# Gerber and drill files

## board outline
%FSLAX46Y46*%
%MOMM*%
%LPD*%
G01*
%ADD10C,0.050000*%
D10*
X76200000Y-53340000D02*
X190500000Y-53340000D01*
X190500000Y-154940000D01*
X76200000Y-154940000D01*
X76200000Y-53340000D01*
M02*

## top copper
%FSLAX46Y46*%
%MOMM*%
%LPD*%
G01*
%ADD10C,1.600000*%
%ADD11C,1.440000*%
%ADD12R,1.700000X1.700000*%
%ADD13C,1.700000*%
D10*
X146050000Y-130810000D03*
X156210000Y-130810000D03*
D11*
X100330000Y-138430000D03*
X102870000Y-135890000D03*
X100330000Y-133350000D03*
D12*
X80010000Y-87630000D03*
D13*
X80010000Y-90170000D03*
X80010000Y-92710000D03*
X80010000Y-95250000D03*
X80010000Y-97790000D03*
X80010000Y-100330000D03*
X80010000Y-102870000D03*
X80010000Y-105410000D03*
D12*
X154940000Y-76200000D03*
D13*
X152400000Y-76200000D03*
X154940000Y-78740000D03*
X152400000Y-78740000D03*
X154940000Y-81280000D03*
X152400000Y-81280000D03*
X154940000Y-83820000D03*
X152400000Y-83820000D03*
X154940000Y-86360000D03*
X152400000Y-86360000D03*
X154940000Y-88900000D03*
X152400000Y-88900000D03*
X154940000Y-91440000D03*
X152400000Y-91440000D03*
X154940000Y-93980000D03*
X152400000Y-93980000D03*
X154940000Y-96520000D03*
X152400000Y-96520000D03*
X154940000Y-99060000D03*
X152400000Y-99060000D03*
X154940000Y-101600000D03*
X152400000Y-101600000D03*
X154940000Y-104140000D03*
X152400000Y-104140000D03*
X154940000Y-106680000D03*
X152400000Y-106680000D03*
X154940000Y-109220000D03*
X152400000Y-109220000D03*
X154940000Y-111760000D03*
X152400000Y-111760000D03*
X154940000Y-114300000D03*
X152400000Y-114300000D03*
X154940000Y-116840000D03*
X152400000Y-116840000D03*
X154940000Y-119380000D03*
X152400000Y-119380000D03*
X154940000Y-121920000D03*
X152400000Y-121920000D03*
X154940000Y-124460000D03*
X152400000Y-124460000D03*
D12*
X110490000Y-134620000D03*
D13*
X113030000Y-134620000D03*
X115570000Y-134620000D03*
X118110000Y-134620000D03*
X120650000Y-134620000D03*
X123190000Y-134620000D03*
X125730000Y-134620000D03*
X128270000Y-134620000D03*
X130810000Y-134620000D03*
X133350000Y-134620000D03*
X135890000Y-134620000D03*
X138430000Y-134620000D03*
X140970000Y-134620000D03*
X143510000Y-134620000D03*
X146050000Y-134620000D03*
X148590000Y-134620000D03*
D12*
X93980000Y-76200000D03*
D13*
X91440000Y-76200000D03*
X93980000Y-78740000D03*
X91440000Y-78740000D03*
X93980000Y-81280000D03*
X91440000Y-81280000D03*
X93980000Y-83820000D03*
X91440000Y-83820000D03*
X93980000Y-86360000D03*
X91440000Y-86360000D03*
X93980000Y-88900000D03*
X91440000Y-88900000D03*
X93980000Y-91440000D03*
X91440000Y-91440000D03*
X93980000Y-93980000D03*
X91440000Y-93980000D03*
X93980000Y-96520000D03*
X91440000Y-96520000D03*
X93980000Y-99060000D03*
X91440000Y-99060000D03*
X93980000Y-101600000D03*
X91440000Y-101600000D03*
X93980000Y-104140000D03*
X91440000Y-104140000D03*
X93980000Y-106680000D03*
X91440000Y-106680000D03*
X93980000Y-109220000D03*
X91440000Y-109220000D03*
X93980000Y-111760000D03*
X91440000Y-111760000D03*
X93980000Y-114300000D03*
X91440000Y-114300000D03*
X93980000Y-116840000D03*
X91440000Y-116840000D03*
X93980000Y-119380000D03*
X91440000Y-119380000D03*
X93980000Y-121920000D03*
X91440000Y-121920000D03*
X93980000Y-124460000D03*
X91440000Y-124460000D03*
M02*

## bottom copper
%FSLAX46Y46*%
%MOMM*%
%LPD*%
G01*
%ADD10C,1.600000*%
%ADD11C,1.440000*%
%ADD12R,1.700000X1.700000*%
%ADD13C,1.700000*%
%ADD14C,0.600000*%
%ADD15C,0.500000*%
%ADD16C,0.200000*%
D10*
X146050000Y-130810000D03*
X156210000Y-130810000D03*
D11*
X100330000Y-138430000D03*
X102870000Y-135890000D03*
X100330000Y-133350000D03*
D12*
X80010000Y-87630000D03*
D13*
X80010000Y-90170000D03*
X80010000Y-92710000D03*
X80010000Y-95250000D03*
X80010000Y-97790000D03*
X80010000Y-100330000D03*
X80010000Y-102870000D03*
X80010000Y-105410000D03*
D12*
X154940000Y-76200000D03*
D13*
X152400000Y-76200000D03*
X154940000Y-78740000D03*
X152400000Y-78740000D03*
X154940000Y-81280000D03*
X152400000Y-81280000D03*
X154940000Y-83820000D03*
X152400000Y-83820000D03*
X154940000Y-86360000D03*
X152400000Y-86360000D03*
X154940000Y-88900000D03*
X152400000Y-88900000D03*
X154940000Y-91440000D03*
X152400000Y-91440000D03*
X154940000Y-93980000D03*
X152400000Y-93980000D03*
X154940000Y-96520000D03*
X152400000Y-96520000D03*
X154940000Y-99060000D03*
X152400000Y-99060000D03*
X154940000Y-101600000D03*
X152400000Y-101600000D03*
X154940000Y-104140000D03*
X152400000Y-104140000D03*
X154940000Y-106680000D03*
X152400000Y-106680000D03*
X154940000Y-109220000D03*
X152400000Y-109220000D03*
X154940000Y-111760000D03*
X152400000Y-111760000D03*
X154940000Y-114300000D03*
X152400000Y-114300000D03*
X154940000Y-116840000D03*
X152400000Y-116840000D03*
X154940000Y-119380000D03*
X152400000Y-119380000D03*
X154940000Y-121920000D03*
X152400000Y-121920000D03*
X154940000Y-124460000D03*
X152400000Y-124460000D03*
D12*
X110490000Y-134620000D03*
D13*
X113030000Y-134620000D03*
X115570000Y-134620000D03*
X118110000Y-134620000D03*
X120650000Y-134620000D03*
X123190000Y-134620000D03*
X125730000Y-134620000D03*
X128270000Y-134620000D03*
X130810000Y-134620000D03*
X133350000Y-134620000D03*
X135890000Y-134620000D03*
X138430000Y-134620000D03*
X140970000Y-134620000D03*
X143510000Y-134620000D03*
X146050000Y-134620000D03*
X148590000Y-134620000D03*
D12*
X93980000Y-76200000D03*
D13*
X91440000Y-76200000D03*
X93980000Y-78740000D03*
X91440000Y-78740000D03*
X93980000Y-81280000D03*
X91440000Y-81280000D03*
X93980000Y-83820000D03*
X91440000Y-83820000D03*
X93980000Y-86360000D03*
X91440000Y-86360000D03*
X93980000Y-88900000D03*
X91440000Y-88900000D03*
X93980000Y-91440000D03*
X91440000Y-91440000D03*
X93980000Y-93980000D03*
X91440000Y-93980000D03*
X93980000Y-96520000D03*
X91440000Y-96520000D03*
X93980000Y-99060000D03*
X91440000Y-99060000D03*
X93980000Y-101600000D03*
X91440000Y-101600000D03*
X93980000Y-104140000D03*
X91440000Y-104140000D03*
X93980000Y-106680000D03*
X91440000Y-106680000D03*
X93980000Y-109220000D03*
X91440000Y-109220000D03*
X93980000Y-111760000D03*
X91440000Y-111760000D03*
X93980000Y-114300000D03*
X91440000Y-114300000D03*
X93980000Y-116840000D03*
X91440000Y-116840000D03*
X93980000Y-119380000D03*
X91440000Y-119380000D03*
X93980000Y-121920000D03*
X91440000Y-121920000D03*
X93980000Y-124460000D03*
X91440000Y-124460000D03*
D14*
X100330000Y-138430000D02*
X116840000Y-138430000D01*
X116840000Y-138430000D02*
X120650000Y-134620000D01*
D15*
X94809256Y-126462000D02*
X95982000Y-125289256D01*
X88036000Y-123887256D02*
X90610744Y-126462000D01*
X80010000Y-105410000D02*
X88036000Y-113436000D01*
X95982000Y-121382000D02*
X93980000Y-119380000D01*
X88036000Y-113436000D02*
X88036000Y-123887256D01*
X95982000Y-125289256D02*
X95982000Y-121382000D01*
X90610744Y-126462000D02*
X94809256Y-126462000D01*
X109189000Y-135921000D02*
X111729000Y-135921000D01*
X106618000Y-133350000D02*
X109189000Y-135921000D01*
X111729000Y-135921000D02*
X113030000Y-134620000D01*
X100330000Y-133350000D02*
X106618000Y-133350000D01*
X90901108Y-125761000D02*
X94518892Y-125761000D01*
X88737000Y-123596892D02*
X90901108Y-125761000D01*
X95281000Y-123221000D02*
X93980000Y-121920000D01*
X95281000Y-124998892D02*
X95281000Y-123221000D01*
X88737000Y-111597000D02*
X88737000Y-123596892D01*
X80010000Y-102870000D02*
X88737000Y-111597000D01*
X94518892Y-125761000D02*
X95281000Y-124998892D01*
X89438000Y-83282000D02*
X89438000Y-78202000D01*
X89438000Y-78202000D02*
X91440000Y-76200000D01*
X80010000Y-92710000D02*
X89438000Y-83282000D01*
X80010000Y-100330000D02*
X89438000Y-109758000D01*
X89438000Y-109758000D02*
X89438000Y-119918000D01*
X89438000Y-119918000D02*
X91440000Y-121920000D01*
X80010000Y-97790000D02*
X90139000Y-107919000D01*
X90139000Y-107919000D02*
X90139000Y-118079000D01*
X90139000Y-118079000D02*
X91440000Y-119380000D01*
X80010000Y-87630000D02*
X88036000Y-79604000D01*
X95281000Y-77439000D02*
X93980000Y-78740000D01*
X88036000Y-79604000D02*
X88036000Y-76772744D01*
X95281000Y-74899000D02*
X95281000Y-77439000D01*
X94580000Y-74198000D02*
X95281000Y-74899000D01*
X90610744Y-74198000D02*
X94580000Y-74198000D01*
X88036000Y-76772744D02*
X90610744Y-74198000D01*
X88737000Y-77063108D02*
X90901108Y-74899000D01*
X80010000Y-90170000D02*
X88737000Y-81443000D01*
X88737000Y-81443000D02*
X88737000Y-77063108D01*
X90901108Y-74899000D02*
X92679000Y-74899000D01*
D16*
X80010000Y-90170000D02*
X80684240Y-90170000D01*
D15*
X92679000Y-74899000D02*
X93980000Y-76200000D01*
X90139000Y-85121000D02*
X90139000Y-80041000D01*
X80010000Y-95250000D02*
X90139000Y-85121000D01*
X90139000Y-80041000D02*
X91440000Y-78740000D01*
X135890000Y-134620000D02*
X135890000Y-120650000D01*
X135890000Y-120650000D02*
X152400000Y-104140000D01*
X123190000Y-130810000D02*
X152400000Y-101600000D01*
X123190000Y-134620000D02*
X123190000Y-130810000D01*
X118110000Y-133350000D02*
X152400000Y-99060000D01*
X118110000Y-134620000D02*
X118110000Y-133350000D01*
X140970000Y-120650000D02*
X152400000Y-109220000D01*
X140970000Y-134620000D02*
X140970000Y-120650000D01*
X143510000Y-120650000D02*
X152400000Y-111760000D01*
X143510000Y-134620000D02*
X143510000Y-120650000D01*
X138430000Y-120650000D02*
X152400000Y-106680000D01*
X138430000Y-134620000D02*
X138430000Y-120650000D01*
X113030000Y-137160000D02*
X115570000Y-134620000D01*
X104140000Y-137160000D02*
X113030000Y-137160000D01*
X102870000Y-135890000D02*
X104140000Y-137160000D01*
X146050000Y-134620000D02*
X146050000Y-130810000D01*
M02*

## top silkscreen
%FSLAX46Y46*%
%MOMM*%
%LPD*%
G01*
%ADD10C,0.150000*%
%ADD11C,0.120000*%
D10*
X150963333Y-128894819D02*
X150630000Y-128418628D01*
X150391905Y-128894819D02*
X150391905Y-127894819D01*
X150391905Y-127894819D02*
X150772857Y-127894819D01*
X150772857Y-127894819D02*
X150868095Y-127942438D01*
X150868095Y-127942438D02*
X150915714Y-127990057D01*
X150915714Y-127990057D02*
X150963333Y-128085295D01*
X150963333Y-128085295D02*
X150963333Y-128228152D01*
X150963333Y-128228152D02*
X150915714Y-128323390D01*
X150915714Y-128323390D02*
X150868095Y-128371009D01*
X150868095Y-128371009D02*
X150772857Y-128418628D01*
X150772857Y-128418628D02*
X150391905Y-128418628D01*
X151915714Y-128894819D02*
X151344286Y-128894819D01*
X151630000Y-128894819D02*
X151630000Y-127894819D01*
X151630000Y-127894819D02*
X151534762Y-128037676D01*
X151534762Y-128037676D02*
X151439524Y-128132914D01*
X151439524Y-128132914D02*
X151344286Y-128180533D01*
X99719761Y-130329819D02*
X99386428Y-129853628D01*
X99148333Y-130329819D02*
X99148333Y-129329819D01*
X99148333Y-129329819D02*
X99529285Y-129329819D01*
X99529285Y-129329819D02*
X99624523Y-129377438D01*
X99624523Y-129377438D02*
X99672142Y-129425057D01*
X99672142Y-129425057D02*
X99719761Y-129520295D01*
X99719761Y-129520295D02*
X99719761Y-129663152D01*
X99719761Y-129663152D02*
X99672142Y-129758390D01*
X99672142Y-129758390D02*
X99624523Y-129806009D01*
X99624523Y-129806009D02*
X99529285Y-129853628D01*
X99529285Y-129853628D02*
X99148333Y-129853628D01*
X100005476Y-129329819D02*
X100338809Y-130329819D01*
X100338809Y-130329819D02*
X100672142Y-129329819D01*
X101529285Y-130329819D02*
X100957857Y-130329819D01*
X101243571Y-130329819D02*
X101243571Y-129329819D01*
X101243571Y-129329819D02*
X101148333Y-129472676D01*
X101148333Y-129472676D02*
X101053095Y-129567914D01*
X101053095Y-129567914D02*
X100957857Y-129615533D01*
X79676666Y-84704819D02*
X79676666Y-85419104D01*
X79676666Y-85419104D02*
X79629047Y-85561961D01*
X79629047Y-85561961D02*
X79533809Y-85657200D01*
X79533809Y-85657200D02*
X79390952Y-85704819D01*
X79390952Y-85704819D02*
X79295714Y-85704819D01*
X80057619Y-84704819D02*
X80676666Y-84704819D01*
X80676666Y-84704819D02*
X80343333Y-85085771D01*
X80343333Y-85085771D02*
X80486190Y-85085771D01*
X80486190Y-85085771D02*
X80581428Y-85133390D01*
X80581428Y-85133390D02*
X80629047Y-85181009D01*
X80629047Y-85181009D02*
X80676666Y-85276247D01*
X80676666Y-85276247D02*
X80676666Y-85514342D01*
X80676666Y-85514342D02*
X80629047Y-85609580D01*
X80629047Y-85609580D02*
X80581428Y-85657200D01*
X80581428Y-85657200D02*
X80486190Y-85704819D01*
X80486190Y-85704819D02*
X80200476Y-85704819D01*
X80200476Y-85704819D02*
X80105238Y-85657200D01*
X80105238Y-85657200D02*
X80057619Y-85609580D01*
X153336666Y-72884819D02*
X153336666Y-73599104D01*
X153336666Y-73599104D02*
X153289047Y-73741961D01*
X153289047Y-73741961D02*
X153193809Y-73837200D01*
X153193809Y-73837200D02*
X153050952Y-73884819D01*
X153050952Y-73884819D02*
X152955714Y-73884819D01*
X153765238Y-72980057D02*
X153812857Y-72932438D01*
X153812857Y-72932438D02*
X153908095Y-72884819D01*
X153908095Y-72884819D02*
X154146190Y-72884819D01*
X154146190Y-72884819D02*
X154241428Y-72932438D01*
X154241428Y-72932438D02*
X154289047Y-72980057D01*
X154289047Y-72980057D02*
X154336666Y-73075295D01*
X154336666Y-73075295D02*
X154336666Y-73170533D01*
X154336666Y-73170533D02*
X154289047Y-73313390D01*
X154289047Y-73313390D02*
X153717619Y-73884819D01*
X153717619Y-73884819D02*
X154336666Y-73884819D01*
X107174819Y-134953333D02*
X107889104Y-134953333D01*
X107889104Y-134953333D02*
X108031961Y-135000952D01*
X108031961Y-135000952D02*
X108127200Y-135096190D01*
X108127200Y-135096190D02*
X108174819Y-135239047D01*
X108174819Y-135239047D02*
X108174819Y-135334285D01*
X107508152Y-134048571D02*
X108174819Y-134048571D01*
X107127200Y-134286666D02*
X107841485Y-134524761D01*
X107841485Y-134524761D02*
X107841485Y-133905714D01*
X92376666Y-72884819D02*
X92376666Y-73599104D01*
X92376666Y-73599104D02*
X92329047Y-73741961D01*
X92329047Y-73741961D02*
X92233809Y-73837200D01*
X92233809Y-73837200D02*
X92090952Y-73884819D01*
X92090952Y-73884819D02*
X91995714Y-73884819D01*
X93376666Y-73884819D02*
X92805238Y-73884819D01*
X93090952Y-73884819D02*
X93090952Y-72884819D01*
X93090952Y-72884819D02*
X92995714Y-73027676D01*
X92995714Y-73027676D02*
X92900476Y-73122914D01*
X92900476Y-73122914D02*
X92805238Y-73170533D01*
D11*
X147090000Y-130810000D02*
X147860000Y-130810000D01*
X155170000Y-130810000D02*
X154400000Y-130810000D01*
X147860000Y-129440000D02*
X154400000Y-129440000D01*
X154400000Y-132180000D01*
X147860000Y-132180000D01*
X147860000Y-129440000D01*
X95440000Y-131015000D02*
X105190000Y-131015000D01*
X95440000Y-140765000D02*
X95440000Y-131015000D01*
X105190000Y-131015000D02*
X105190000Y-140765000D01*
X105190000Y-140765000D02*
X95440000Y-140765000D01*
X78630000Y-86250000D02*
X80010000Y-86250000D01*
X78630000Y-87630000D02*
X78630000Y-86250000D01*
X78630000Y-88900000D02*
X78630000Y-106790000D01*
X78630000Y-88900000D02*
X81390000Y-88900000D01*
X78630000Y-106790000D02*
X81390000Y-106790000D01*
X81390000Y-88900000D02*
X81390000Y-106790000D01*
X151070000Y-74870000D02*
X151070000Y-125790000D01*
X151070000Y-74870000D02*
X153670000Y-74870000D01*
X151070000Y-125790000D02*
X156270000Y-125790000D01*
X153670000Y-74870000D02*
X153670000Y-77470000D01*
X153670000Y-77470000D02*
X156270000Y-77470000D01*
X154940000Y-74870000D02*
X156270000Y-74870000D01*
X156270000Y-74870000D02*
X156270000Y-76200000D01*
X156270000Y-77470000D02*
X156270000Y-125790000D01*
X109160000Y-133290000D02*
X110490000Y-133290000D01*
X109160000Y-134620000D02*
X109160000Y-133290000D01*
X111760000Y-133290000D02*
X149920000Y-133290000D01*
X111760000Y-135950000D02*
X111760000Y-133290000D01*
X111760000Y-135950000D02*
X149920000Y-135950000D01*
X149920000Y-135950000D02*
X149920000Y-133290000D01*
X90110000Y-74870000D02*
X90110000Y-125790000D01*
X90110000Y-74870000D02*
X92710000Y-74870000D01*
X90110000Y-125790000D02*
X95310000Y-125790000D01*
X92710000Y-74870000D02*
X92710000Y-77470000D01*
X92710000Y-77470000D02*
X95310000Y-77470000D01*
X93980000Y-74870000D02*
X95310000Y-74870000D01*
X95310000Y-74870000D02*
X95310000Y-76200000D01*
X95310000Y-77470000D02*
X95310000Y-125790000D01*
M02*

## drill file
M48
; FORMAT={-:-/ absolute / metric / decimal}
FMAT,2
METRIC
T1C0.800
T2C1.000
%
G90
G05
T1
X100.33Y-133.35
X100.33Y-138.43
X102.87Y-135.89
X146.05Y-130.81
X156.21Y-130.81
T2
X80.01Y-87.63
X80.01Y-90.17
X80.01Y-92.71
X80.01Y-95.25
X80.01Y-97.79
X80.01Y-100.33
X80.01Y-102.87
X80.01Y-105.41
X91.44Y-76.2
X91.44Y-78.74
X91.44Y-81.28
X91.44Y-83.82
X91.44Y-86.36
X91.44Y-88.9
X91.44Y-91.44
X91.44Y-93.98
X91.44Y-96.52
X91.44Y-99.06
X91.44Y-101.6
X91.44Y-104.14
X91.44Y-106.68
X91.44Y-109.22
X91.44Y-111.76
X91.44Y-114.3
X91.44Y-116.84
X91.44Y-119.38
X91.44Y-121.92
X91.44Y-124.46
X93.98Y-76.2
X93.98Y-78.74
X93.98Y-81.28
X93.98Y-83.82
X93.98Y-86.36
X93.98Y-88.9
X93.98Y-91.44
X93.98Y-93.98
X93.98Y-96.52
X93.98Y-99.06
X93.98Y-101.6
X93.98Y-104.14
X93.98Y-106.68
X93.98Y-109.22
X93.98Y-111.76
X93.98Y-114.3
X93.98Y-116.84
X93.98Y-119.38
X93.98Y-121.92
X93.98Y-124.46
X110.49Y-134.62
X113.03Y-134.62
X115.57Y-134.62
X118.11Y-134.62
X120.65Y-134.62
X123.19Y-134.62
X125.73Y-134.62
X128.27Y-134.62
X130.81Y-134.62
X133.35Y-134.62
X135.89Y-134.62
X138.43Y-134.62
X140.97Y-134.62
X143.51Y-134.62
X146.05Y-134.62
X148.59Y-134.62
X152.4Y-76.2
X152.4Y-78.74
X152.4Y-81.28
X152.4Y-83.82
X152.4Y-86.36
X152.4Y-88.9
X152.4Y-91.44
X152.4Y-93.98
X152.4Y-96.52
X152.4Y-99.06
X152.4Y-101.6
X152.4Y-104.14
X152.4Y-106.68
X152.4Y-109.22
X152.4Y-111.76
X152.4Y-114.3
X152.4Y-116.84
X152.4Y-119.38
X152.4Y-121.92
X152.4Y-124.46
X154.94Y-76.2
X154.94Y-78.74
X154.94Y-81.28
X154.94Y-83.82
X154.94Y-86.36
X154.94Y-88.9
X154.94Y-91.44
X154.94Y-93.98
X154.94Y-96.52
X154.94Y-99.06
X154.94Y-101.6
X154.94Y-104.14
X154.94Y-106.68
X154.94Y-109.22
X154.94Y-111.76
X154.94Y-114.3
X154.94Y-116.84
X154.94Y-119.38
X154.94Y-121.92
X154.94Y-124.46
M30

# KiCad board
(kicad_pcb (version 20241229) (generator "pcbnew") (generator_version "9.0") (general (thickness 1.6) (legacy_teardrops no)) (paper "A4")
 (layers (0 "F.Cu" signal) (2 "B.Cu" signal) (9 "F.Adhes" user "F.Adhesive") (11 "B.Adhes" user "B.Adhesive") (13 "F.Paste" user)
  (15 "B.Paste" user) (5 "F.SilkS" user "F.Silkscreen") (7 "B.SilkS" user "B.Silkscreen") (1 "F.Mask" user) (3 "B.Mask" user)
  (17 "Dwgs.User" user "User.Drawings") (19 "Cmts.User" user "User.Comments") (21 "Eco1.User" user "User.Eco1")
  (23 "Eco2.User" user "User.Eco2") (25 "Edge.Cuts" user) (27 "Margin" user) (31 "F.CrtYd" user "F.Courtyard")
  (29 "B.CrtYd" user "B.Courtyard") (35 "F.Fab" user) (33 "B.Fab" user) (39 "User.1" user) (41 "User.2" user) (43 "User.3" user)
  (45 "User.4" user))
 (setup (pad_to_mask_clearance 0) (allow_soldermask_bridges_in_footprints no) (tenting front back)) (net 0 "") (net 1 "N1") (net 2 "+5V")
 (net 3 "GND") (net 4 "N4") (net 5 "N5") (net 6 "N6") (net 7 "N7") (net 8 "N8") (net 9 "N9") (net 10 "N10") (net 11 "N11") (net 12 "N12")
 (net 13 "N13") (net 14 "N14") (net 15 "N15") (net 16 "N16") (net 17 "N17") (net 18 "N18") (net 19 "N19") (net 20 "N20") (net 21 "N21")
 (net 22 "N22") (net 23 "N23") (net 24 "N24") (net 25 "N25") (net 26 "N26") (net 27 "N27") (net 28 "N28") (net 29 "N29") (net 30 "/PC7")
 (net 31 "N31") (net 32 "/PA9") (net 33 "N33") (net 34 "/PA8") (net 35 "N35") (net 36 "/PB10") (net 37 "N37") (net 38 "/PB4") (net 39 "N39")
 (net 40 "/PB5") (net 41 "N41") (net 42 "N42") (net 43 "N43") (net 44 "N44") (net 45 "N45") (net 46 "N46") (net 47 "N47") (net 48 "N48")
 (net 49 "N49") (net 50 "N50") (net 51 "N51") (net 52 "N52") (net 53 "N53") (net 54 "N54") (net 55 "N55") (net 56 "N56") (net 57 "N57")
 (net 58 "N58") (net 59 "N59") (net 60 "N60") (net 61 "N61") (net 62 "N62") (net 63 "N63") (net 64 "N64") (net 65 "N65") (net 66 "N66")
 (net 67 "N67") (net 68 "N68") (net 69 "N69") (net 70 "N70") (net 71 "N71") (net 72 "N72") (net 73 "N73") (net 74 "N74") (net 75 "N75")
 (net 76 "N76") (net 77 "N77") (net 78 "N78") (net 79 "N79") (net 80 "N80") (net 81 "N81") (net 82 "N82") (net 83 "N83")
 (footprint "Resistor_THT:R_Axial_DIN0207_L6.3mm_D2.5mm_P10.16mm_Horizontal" (layer "F.Cu") (at 146.05 130.81)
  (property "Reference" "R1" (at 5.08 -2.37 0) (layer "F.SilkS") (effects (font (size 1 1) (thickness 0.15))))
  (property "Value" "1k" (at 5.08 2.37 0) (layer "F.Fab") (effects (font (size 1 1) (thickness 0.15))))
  (fp_line (start 1.04 0) (end 1.81 0) (stroke (width 0.12) (type solid)) (layer "F.SilkS"))
  (fp_line (start 9.12 0) (end 8.35 0) (stroke (width 0.12) (type solid)) (layer "F.SilkS"))
  (fp_rect (start 1.81 -1.37) (end 8.35 1.37) (stroke (width 0.12) (type solid)) (fill no) (layer "F.SilkS"))
  (pad "1" thru_hole circle (at 0 0) (size 1.6 1.6) (drill 0.8) (layers "*.Cu" "*.Mask") (remove_unused_layers no) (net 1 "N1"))
  (pad "2" thru_hole circle (at 10.16 0) (size 1.6 1.6) (drill 0.8) (layers "*.Cu" "*.Mask") (remove_unused_layers no) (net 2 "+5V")))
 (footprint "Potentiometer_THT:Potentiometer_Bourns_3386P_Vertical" (layer "F.Cu") (at 100.33 138.43)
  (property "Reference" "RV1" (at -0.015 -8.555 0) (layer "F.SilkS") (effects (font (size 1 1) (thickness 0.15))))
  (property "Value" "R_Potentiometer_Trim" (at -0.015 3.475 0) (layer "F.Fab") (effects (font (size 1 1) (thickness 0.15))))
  (fp_line (start -4.89 -7.415) (end 4.86 -7.415) (stroke (width 0.12) (type solid)) (layer "F.SilkS"))
  (fp_line (start -4.89 2.335) (end -4.89 -7.415) (stroke (width 0.12) (type solid)) (layer "F.SilkS"))
  (fp_line (start 4.86 -7.415) (end 4.86 2.335) (stroke (width 0.12) (type solid)) (layer "F.SilkS"))
  (fp_line (start 4.86 2.335) (end -4.89 2.335) (stroke (width 0.12) (type solid)) (layer "F.SilkS"))
  (pad "1" thru_hole circle (at 0 0) (size 1.44 1.44) (drill 0.8) (layers "*.Cu" "*.Mask") (remove_unused_layers no) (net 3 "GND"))
  (pad "2" thru_hole circle (at 2.54 -2.54) (size 1.44 1.44) (drill 0.8) (layers "*.Cu" "*.Mask") (remove_unused_layers no) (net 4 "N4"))
  (pad "3" thru_hole circle (at 0 -5.08) (size 1.44 1.44) (drill 0.8) (layers "*.Cu" "*.Mask") (remove_unused_layers no) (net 2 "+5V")))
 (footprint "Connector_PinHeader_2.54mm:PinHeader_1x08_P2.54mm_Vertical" (layer "F.Cu") (at 80.01 87.63)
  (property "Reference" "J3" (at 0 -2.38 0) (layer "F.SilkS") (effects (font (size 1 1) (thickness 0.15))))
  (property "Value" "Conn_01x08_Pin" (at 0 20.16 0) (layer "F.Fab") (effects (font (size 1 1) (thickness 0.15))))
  (fp_line (start -1.38 -1.38) (end 0 -1.38) (stroke (width 0.12) (type solid)) (layer "F.SilkS"))
  (fp_line (start -1.38 0) (end -1.38 -1.38) (stroke (width 0.12) (type solid)) (layer "F.SilkS"))
  (fp_line (start -1.38 1.27) (end -1.38 19.16) (stroke (width 0.12) (type solid)) (layer "F.SilkS"))
  (fp_line (start -1.38 1.27) (end 1.38 1.27) (stroke (width 0.12) (type solid)) (layer "F.SilkS"))
  (fp_line (start -1.38 19.16) (end 1.38 19.16) (stroke (width 0.12) (type solid)) (layer "F.SilkS"))
  (fp_line (start 1.38 1.27) (end 1.38 19.16) (stroke (width 0.12) (type solid)) (layer "F.SilkS"))
  (pad "1" thru_hole rect (at 0 0) (size 1.7 1.7) (drill 1) (layers "*.Cu" "*.Mask") (remove_unused_layers no) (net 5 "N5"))
  (pad "2" thru_hole circle (at 0 2.54) (size 1.7 1.7) (drill 1) (layers "*.Cu" "*.Mask") (remove_unused_layers no) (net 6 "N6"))
  (pad "3" thru_hole circle (at 0 5.08) (size 1.7 1.7) (drill 1) (layers "*.Cu" "*.Mask") (remove_unused_layers no) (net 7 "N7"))
  (pad "4" thru_hole circle (at 0 7.62) (size 1.7 1.7) (drill 1) (layers "*.Cu" "*.Mask") (remove_unused_layers no) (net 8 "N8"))
  (pad "5" thru_hole circle (at 0 10.16) (size 1.7 1.7) (drill 1) (layers "*.Cu" "*.Mask") (remove_unused_layers no) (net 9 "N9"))
  (pad "6" thru_hole circle (at 0 12.7) (size 1.7 1.7) (drill 1) (layers "*.Cu" "*.Mask") (remove_unused_layers no) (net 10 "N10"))
  (pad "7" thru_hole circle (at 0 15.24) (size 1.7 1.7) (drill 1) (layers "*.Cu" "*.Mask") (remove_unused_layers no) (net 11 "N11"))
  (pad "8" thru_hole circle (at 0 17.78) (size 1.7 1.7) (drill 1) (layers "*.Cu" "*.Mask") (remove_unused_layers no) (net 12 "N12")))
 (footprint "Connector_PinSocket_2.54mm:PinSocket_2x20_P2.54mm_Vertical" (layer "F.Cu") (at 154.94 76.2)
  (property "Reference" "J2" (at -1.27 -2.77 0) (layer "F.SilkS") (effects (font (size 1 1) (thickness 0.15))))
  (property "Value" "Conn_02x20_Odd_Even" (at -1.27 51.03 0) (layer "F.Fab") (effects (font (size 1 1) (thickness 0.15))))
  (fp_line (start -3.87 -1.33) (end -3.87 49.59) (stroke (width 0.12) (type solid)) (layer "F.SilkS"))
  (fp_line (start -3.87 -1.33) (end -1.27 -1.33) (stroke (width 0.12) (type solid)) (layer "F.SilkS"))
  (fp_line (start -3.87 49.59) (end 1.33 49.59) (stroke (width 0.12) (type solid)) (layer "F.SilkS"))
  (fp_line (start -1.27 -1.33) (end -1.27 1.27) (stroke (width 0.12) (type solid)) (layer "F.SilkS"))
  (fp_line (start -1.27 1.27) (end 1.33 1.27) (stroke (width 0.12) (type solid)) (layer "F.SilkS"))
  (fp_line (start 0 -1.33) (end 1.33 -1.33) (stroke (width 0.12) (type solid)) (layer "F.SilkS"))
  (fp_line (start 1.33 -1.33) (end 1.33 0) (stroke (width 0.12) (type solid)) (layer "F.SilkS"))
  (fp_line (start 1.33 1.27) (end 1.33 49.59) (stroke (width 0.12) (type solid)) (layer "F.SilkS"))
  (pad "1" thru_hole rect (at 0 0) (size 1.7 1.7) (drill 1) (layers "*.Cu" "*.Mask") (remove_unused_layers no) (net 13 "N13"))
  (pad "2" thru_hole circle (at -2.54 0) (size 1.7 1.7) (drill 1) (layers "*.Cu" "*.Mask") (remove_unused_layers no) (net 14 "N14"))
  (pad "3" thru_hole circle (at 0 2.54) (size 1.7 1.7) (drill 1) (layers "*.Cu" "*.Mask") (remove_unused_layers no) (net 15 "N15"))
  (pad "4" thru_hole circle (at -2.54 2.54) (size 1.7 1.7) (drill 1) (layers "*.Cu" "*.Mask") (remove_unused_layers no) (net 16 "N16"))
  (pad "5" thru_hole circle (at 0 5.08) (size 1.7 1.7) (drill 1) (layers "*.Cu" "*.Mask") (remove_unused_layers no) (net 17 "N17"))
  (pad "6" thru_hole circle (at -2.54 5.08) (size 1.7 1.7) (drill 1) (layers "*.Cu" "*.Mask") (remove_unused_layers no) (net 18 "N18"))
  (pad "7" thru_hole circle (at 0 7.62) (size 1.7 1.7) (drill 1) (layers "*.Cu" "*.Mask") (remove_unused_layers no) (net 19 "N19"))
  (pad "8" thru_hole circle (at -2.54 7.62) (size 1.7 1.7) (drill 1) (layers "*.Cu" "*.Mask") (remove_unused_layers no) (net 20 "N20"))
  (pad "9" thru_hole circle (at 0 10.16) (size 1.7 1.7) (drill 1) (layers "*.Cu" "*.Mask") (remove_unused_layers no) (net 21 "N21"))
  (pad "10" thru_hole circle (at -2.54 10.16) (size 1.7 1.7) (drill 1) (layers "*.Cu" "*.Mask") (remove_unused_layers no) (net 3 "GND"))
  (pad "11" thru_hole circle (at 0 12.7) (size 1.7 1.7) (drill 1) (layers "*.Cu" "*.Mask") (remove_unused_layers no) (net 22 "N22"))
  (pad "12" thru_hole circle (at -2.54 12.7) (size 1.7 1.7) (drill 1) (layers "*.Cu" "*.Mask") (remove_unused_layers no) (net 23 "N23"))
  (pad "13" thru_hole circle (at 0 15.24) (size 1.7 1.7) (drill 1) (layers "*.Cu" "*.Mask") (remove_unused_layers no) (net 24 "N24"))
  (pad "14" thru_hole circle (at -2.54 15.24) (size 1.7 1.7) (drill 1) (layers "*.Cu" "*.Mask") (remove_unused_layers no) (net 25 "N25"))
  (pad "15" thru_hole circle (at 0 17.78) (size 1.7 1.7) (drill 1) (layers "*.Cu" "*.Mask") (remove_unused_layers no) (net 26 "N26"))
  (pad "16" thru_hole circle (at -2.54 17.78) (size 1.7 1.7) (drill 1) (layers "*.Cu" "*.Mask") (remove_unused_layers no) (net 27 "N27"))
  (pad "17" thru_hole circle (at 0 20.32) (size 1.7 1.7) (drill 1) (layers "*.Cu" "*.Mask") (remove_unused_layers no) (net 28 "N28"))
  (pad "18" thru_hole circle (at -2.54 20.32) (size 1.7 1.7) (drill 1) (layers "*.Cu" "*.Mask") (remove_unused_layers no) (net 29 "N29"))
  (pad "19" thru_hole circle (at 0 22.86) (size 1.7 1.7) (drill 1) (layers "*.Cu" "*.Mask") (remove_unused_layers no) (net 3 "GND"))
  (pad "20" thru_hole circle (at -2.54 22.86) (size 1.7 1.7) (drill 1) (layers "*.Cu" "*.Mask") (remove_unused_layers no) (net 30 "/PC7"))
  (pad "21" thru_hole circle (at 0 25.4) (size 1.7 1.7) (drill 1) (layers "*.Cu" "*.Mask") (remove_unused_layers no) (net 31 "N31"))
  (pad "22" thru_hole circle (at -2.54 25.4) (size 1.7 1.7) (drill 1) (layers "*.Cu" "*.Mask") (remove_unused_layers no) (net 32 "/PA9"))
  (pad "23" thru_hole circle (at 0 27.94) (size 1.7 1.7) (drill 1) (layers "*.Cu" "*.Mask") (remove_unused_layers no) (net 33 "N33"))
  (pad "24" thru_hole circle (at -2.54 27.94) (size 1.7 1.7) (drill 1) (layers "*.Cu" "*.Mask") (remove_unused_layers no) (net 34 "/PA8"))
  (pad "25" thru_hole circle (at 0 30.48) (size 1.7 1.7) (drill 1) (layers "*.Cu" "*.Mask") (remove_unused_layers no) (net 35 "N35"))
  (pad "26" thru_hole circle (at -2.54 30.48) (size 1.7 1.7) (drill 1) (layers "*.Cu" "*.Mask") (remove_unused_layers no) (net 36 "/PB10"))
  (pad "27" thru_hole circle (at 0 33.02) (size 1.7 1.7) (drill 1) (layers "*.Cu" "*.Mask") (remove_unused_layers no) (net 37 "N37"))
  (pad "28" thru_hole circle (at -2.54 33.02) (size 1.7 1.7) (drill 1) (layers "*.Cu" "*.Mask") (remove_unused_layers no) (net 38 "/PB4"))
  (pad "29" thru_hole circle (at 0 35.56) (size 1.7 1.7) (drill 1) (layers "*.Cu" "*.Mask") (remove_unused_layers no) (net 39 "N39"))
  (pad "30" thru_hole circle (at -2.54 35.56) (size 1.7 1.7) (drill 1) (layers "*.Cu" "*.Mask") (remove_unused_layers no) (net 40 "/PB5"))
  (pad "31" thru_hole circle (at 0 38.1) (size 1.7 1.7) (drill 1) (layers "*.Cu" "*.Mask") (remove_unused_layers no) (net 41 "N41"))
  (pad "32" thru_hole circle (at -2.54 38.1) (size 1.7 1.7) (drill 1) (layers "*.Cu" "*.Mask") (remove_unused_layers no) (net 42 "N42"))
  (pad "33" thru_hole circle (at 0 40.64) (size 1.7 1.7) (drill 1) (layers "*.Cu" "*.Mask") (remove_unused_layers no) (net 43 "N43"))
  (pad "34" thru_hole circle (at -2.54 40.64) (size 1.7 1.7) (drill 1) (layers "*.Cu" "*.Mask") (remove_unused_layers no) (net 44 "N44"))
  (pad "35" thru_hole circle (at 0 43.18) (size 1.7 1.7) (drill 1) (layers "*.Cu" "*.Mask") (remove_unused_layers no) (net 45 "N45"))
  (pad "36" thru_hole circle (at -2.54 43.18) (size 1.7 1.7) (drill 1) (layers "*.Cu" "*.Mask") (remove_unused_layers no) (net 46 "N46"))
  (pad "37" thru_hole circle (at 0 45.72) (size 1.7 1.7) (drill 1) (layers "*.Cu" "*.Mask") (remove_unused_layers no) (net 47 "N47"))
  (pad "38" thru_hole circle (at -2.54 45.72) (size 1.7 1.7) (drill 1) (layers "*.Cu" "*.Mask") (remove_unused_layers no) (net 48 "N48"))
  (pad "39" thru_hole circle (at 0 48.26) (size 1.7 1.7) (drill 1) (layers "*.Cu" "*.Mask") (remove_unused_layers no) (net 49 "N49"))
  (pad "40" thru_hole circle (at -2.54 48.26) (size 1.7 1.7) (drill 1) (layers "*.Cu" "*.Mask") (remove_unused_layers no) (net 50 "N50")))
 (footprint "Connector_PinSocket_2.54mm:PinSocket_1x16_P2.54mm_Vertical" (layer "F.Cu") (at 110.49 134.62 90)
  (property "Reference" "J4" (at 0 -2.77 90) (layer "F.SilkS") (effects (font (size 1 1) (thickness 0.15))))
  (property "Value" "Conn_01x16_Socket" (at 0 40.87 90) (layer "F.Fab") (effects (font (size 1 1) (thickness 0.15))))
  (fp_line (start 1.33 -1.33) (end 1.33 0) (stroke (width 0.12) (type solid)) (layer "F.SilkS"))
  (fp_line (start 0 -1.33) (end 1.33 -1.33) (stroke (width 0.12) (type solid)) (layer "F.SilkS"))
  (fp_line (start 1.33 1.27) (end 1.33 39.43) (stroke (width 0.12) (type solid)) (layer "F.SilkS"))
  (fp_line (start -1.33 1.27) (end 1.33 1.27) (stroke (width 0.12) (type solid)) (layer "F.SilkS"))
  (fp_line (start -1.33 1.27) (end -1.33 39.43) (stroke (width 0.12) (type solid)) (layer "F.SilkS"))
  (fp_line (start -1.33 39.43) (end 1.33 39.43) (stroke (width 0.12) (type solid)) (layer "F.SilkS"))
  (pad "1" thru_hole rect (at 0 0 90) (size 1.7 1.7) (drill 1) (layers "*.Cu" "*.Mask") (remove_unused_layers no) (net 3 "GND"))
  (pad "2" thru_hole circle (at 0 2.54 90) (size 1.7 1.7) (drill 1) (layers "*.Cu" "*.Mask") (remove_unused_layers no) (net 2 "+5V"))
  (pad "3" thru_hole circle (at 0 5.08 90) (size 1.7 1.7) (drill 1) (layers "*.Cu" "*.Mask") (remove_unused_layers no) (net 4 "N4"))
  (pad "4" thru_hole circle (at 0 7.62 90) (size 1.7 1.7) (drill 1) (layers "*.Cu" "*.Mask") (remove_unused_layers no) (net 30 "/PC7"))
  (pad "5" thru_hole circle (at 0 10.16 90) (size 1.7 1.7) (drill 1) (layers "*.Cu" "*.Mask") (remove_unused_layers no) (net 3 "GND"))
  (pad "6" thru_hole circle (at 0 12.7 90) (size 1.7 1.7) (drill 1) (layers "*.Cu" "*.Mask") (remove_unused_layers no) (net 32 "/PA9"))
  (pad "7" thru_hole circle (at 0 15.24 90) (size 1.7 1.7) (drill 1) (layers "*.Cu" "*.Mask") (remove_unused_layers no) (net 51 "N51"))
  (pad "8" thru_hole circle (at 0 17.78 90) (size 1.7 1.7) (drill 1) (layers "*.Cu" "*.Mask") (remove_unused_layers no) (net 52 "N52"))
  (pad "9" thru_hole circle (at 0 20.32 90) (size 1.7 1.7) (drill 1) (layers "*.Cu" "*.Mask") (remove_unused_layers no) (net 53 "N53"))
  (pad "10" thru_hole circle (at 0 22.86 90) (size 1.7 1.7) (drill 1) (layers "*.Cu" "*.Mask") (remove_unused_layers no) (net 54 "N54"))
  (pad "11" thru_hole circle (at 0 25.4 90) (size 1.7 1.7) (drill 1) (layers "*.Cu" "*.Mask") (remove_unused_layers no) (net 34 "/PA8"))
  (pad "12" thru_hole circle (at 0 27.94 90) (size 1.7 1.7) (drill 1) (layers "*.Cu" "*.Mask") (remove_unused_layers no) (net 36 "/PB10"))
  (pad "13" thru_hole circle (at 0 30.48 90) (size 1.7 1.7) (drill 1) (layers "*.Cu" "*.Mask") (remove_unused_layers no) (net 38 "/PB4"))
  (pad "14" thru_hole circle (at 0 33.02 90) (size 1.7 1.7) (drill 1) (layers "*.Cu" "*.Mask") (remove_unused_layers no) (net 40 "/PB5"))
  (pad "15" thru_hole circle (at 0 35.56 90) (size 1.7 1.7) (drill 1) (layers "*.Cu" "*.Mask") (remove_unused_layers no) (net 1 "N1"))
  (pad "16" thru_hole circle (at 0 38.1 90) (size 1.7 1.7) (drill 1) (layers "*.Cu" "*.Mask") (remove_unused_layers no) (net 3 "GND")))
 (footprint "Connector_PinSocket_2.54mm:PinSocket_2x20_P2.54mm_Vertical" (layer "F.Cu") (at 93.98 76.2)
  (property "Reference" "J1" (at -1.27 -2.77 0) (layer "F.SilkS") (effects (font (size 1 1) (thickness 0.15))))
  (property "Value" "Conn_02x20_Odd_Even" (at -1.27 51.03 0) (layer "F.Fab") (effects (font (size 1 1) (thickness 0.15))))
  (fp_line (start -3.87 -1.33) (end -3.87 49.59) (stroke (width 0.12) (type solid)) (layer "F.SilkS"))
  (fp_line (start -3.87 -1.33) (end -1.27 -1.33) (stroke (width 0.12) (type solid)) (layer "F.SilkS"))
  (fp_line (start -3.87 49.59) (end 1.33 49.59) (stroke (width 0.12) (type solid)) (layer "F.SilkS"))
  (fp_line (start -1.27 -1.33) (end -1.27 1.27) (stroke (width 0.12) (type solid)) (layer "F.SilkS"))
  (fp_line (start -1.27 1.27) (end 1.33 1.27) (stroke (width 0.12) (type solid)) (layer "F.SilkS"))
  (fp_line (start 0 -1.33) (end 1.33 -1.33) (stroke (width 0.12) (type solid)) (layer "F.SilkS"))
  (fp_line (start 1.33 -1.33) (end 1.33 0) (stroke (width 0.12) (type solid)) (layer "F.SilkS"))
  (fp_line (start 1.33 1.27) (end 1.33 49.59) (stroke (width 0.12) (type solid)) (layer "F.SilkS"))
  (pad "1" thru_hole rect (at 0 0) (size 1.7 1.7) (drill 1) (layers "*.Cu" "*.Mask") (remove_unused_layers no) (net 6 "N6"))
  (pad "2" thru_hole circle (at -2.54 0) (size 1.7 1.7) (drill 1) (layers "*.Cu" "*.Mask") (remove_unused_layers no) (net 7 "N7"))
  (pad "3" thru_hole circle (at 0 2.54) (size 1.7 1.7) (drill 1) (layers "*.Cu" "*.Mask") (remove_unused_layers no) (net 5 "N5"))
  (pad "4" thru_hole circle (at -2.54 2.54) (size 1.7 1.7) (drill 1) (layers "*.Cu" "*.Mask") (remove_unused_layers no) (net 8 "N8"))
  (pad "5" thru_hole circle (at 0 5.08) (size 1.7 1.7) (drill 1) (layers "*.Cu" "*.Mask") (remove_unused_layers no) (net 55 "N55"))
  (pad "6" thru_hole circle (at -2.54 5.08) (size 1.7 1.7) (drill 1) (layers "*.Cu" "*.Mask") (remove_unused_layers no) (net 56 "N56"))
  (pad "7" thru_hole circle (at 0 7.62) (size 1.7 1.7) (drill 1) (layers "*.Cu" "*.Mask") (remove_unused_layers no) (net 3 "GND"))
  (pad "8" thru_hole circle (at -2.54 7.62) (size 1.7 1.7) (drill 1) (layers "*.Cu" "*.Mask") (remove_unused_layers no) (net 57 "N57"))
  (pad "9" thru_hole circle (at 0 10.16) (size 1.7 1.7) (drill 1) (layers "*.Cu" "*.Mask") (remove_unused_layers no) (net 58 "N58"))
  (pad "10" thru_hole circle (at -2.54 10.16) (size 1.7 1.7) (drill 1) (layers "*.Cu" "*.Mask") (remove_unused_layers no) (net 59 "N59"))
  (pad "11" thru_hole circle (at 0 12.7) (size 1.7 1.7) (drill 1) (layers "*.Cu" "*.Mask") (remove_unused_layers no) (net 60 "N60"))
  (pad "12" thru_hole circle (at -2.54 12.7) (size 1.7 1.7) (drill 1) (layers "*.Cu" "*.Mask") (remove_unused_layers no) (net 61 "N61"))
  (pad "13" thru_hole circle (at 0 15.24) (size 1.7 1.7) (drill 1) (layers "*.Cu" "*.Mask") (remove_unused_layers no) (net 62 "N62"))
  (pad "14" thru_hole circle (at -2.54 15.24) (size 1.7 1.7) (drill 1) (layers "*.Cu" "*.Mask") (remove_unused_layers no) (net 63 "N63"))
  (pad "15" thru_hole circle (at 0 17.78) (size 1.7 1.7) (drill 1) (layers "*.Cu" "*.Mask") (remove_unused_layers no) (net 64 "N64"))
  (pad "16" thru_hole circle (at -2.54 17.78) (size 1.7 1.7) (drill 1) (layers "*.Cu" "*.Mask") (remove_unused_layers no) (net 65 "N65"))
  (pad "17" thru_hole circle (at 0 20.32) (size 1.7 1.7) (drill 1) (layers "*.Cu" "*.Mask") (remove_unused_layers no) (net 2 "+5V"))
  (pad "18" thru_hole circle (at -2.54 20.32) (size 1.7 1.7) (drill 1) (layers "*.Cu" "*.Mask") (remove_unused_layers no) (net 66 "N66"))
  (pad "19" thru_hole circle (at 0 22.86) (size 1.7 1.7) (drill 1) (layers "*.Cu" "*.Mask") (remove_unused_layers no) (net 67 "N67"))
  (pad "20" thru_hole circle (at -2.54 22.86) (size 1.7 1.7) (drill 1) (layers "*.Cu" "*.Mask") (remove_unused_layers no) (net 3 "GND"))
  (pad "21" thru_hole circle (at 0 25.4) (size 1.7 1.7) (drill 1) (layers "*.Cu" "*.Mask") (remove_unused_layers no) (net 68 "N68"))
  (pad "22" thru_hole circle (at -2.54 25.4) (size 1.7 1.7) (drill 1) (layers "*.Cu" "*.Mask") (remove_unused_layers no) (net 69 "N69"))
  (pad "23" thru_hole circle (at 0 27.94) (size 1.7 1.7) (drill 1) (layers "*.Cu" "*.Mask") (remove_unused_layers no) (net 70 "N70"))
  (pad "24" thru_hole circle (at -2.54 27.94) (size 1.7 1.7) (drill 1) (layers "*.Cu" "*.Mask") (remove_unused_layers no) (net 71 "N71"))
  (pad "25" thru_hole circle (at 0 30.48) (size 1.7 1.7) (drill 1) (layers "*.Cu" "*.Mask") (remove_unused_layers no) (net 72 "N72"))
  (pad "26" thru_hole circle (at -2.54 30.48) (size 1.7 1.7) (drill 1) (layers "*.Cu" "*.Mask") (remove_unused_layers no) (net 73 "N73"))
  (pad "27" thru_hole circle (at 0 33.02) (size 1.7 1.7) (drill 1) (layers "*.Cu" "*.Mask") (remove_unused_layers no) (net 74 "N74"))
  (pad "28" thru_hole circle (at -2.54 33.02) (size 1.7 1.7) (drill 1) (layers "*.Cu" "*.Mask") (remove_unused_layers no) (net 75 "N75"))
  (pad "29" thru_hole circle (at 0 35.56) (size 1.7 1.7) (drill 1) (layers "*.Cu" "*.Mask") (remove_unused_layers no) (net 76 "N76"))
  (pad "30" thru_hole circle (at -2.54 35.56) (size 1.7 1.7) (drill 1) (layers "*.Cu" "*.Mask") (remove_unused_layers no) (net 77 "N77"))
  (pad "31" thru_hole circle (at 0 38.1) (size 1.7 1.7) (drill 1) (layers "*.Cu" "*.Mask") (remove_unused_layers no) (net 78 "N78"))
  (pad "32" thru_hole circle (at -2.54 38.1) (size 1.7 1.7) (drill 1) (layers "*.Cu" "*.Mask") (remove_unused_layers no) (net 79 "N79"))
  (pad "33" thru_hole circle (at 0 40.64) (size 1.7 1.7) (drill 1) (layers "*.Cu" "*.Mask") (remove_unused_layers no) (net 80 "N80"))
  (pad "34" thru_hole circle (at -2.54 40.64) (size 1.7 1.7) (drill 1) (layers "*.Cu" "*.Mask") (remove_unused_layers no) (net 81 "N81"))
  (pad "35" thru_hole circle (at 0 43.18) (size 1.7 1.7) (drill 1) (layers "*.Cu" "*.Mask") (remove_unused_layers no) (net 12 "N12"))
  (pad "36" thru_hole circle (at -2.54 43.18) (size 1.7 1.7) (drill 1) (layers "*.Cu" "*.Mask") (remove_unused_layers no) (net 9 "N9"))
  (pad "37" thru_hole circle (at 0 45.72) (size 1.7 1.7) (drill 1) (layers "*.Cu" "*.Mask") (remove_unused_layers no) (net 11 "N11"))
  (pad "38" thru_hole circle (at -2.54 45.72) (size 1.7 1.7) (drill 1) (layers "*.Cu" "*.Mask") (remove_unused_layers no) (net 10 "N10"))
  (pad "39" thru_hole circle (at 0 48.26) (size 1.7 1.7) (drill 1) (layers "*.Cu" "*.Mask") (remove_unused_layers no) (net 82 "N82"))
  (pad "40" thru_hole circle (at -2.54 48.26) (size 1.7 1.7) (drill 1) (layers "*.Cu" "*.Mask") (remove_unused_layers no) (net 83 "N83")))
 (gr_rect (start 76.2 53.34) (end 190.5 154.94) (stroke (width 0.05) (type default)) (fill no) (layer "Edge.Cuts"))
 (segment (start 100.33 138.43) (end 116.84 138.43) (width 0.6) (layer "B.Cu") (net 3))
 (segment (start 116.84 138.43) (end 120.65 134.62) (width 0.6) (layer "B.Cu") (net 3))
 (segment (start 94.809256 126.462) (end 95.982 125.289256) (width 0.5) (layer "B.Cu") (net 12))
 (segment (start 88.036 123.887256) (end 90.610744 126.462) (width 0.5) (layer "B.Cu") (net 12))
 (segment (start 80.01 105.41) (end 88.036 113.436) (width 0.5) (layer "B.Cu") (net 12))
 (segment (start 95.982 121.382) (end 93.98 119.38) (width 0.5) (layer "B.Cu") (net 12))
 (segment (start 88.036 113.436) (end 88.036 123.887256) (width 0.5) (layer "B.Cu") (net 12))
 (segment (start 95.982 125.289256) (end 95.982 121.382) (width 0.5) (layer "B.Cu") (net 12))
 (segment (start 90.610744 126.462) (end 94.809256 126.462) (width 0.5) (layer "B.Cu") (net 12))
 (segment (start 109.189 135.921) (end 111.729 135.921) (width 0.5) (layer "B.Cu") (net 2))
 (segment (start 106.618 133.35) (end 109.189 135.921) (width 0.5) (layer "B.Cu") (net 2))
 (segment (start 111.729 135.921) (end 113.03 134.62) (width 0.5) (layer "B.Cu") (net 2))
 (segment (start 100.33 133.35) (end 106.618 133.35) (width 0.5) (layer "B.Cu") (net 2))
 (segment (start 90.901108 125.761) (end 94.518892 125.761) (width 0.5) (layer "B.Cu") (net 11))
 (segment (start 88.737 123.596892) (end 90.901108 125.761) (width 0.5) (layer "B.Cu") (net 11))
 (segment (start 95.281 123.221) (end 93.98 121.92) (width 0.5) (layer "B.Cu") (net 11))
 (segment (start 95.281 124.998892) (end 95.281 123.221) (width 0.5) (layer "B.Cu") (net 11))
 (segment (start 88.737 111.597) (end 88.737 123.596892) (width 0.5) (layer "B.Cu") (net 11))
 (segment (start 80.01 102.87) (end 88.737 111.597) (width 0.5) (layer "B.Cu") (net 11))
 (segment (start 94.518892 125.761) (end 95.281 124.998892) (width 0.5) (layer "B.Cu") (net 11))
 (segment (start 89.438 83.282) (end 89.438 78.202) (width 0.5) (layer "B.Cu") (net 7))
 (segment (start 89.438 78.202) (end 91.44 76.2) (width 0.5) (layer "B.Cu") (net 7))
 (segment (start 80.01 92.71) (end 89.438 83.282) (width 0.5) (layer "B.Cu") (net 7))
 (segment (start 80.01 100.33) (end 89.438 109.758) (width 0.5) (layer "B.Cu") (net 10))
 (segment (start 89.438 109.758) (end 89.438 119.918) (width 0.5) (layer "B.Cu") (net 10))
 (segment (start 89.438 119.918) (end 91.44 121.92) (width 0.5) (layer "B.Cu") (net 10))
 (segment (start 80.01 97.79) (end 90.139 107.919) (width 0.5) (layer "B.Cu") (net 9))
 (segment (start 90.139 107.919) (end 90.139 118.079) (width 0.5) (layer "B.Cu") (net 9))
 (segment (start 90.139 118.079) (end 91.44 119.38) (width 0.5) (layer "B.Cu") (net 9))
 (segment (start 80.01 87.63) (end 88.036 79.604) (width 0.5) (layer "B.Cu") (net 5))
 (segment (start 95.281 77.439) (end 93.98 78.74) (width 0.5) (layer "B.Cu") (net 5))
 (segment (start 88.036 79.604) (end 88.036 76.772744) (width 0.5) (layer "B.Cu") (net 5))
 (segment (start 95.281 74.899) (end 95.281 77.439) (width 0.5) (layer "B.Cu") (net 5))
 (segment (start 94.58 74.198) (end 95.281 74.899) (width 0.5) (layer "B.Cu") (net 5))
 (segment (start 90.610744 74.198) (end 94.58 74.198) (width 0.5) (layer "B.Cu") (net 5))
 (segment (start 88.036 76.772744) (end 90.610744 74.198) (width 0.5) (layer "B.Cu") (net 5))
 (segment (start 88.737 77.063108) (end 90.901108 74.899) (width 0.5) (layer "B.Cu") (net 6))
 (segment (start 80.01 90.17) (end 88.737 81.443) (width 0.5) (layer "B.Cu") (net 6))
 (segment (start 88.737 81.443) (end 88.737 77.063108) (width 0.5) (layer "B.Cu") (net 6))
 (segment (start 90.901108 74.899) (end 92.679 74.899) (width 0.5) (layer "B.Cu") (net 6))
 (segment (start 80.01 90.17) (end 80.68424 90.17) (width 0.2) (layer "B.Cu") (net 6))
 (segment (start 92.679 74.899) (end 93.98 76.2) (width 0.5) (layer "B.Cu") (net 6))
 (segment (start 90.139 85.121) (end 90.139 80.041) (width 0.5) (layer "B.Cu") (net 8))
 (segment (start 80.01 95.25) (end 90.139 85.121) (width 0.5) (layer "B.Cu") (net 8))
 (segment (start 90.139 80.041) (end 91.44 78.74) (width 0.5) (layer "B.Cu") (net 8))
 (segment (start 135.89 134.62) (end 135.89 120.65) (width 0.5) (layer "B.Cu") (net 34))
 (segment (start 135.89 120.65) (end 152.4 104.14) (width 0.5) (layer "B.Cu") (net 34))
 (segment (start 123.19 130.81) (end 152.4 101.6) (width 0.5) (layer "B.Cu") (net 32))
 (segment (start 123.19 134.62) (end 123.19 130.81) (width 0.5) (layer "B.Cu") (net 32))
 (segment (start 118.11 133.35) (end 152.4 99.06) (width 0.5) (layer "B.Cu") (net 30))
 (segment (start 118.11 134.62) (end 118.11 133.35) (width 0.5) (layer "B.Cu") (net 30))
 (segment (start 140.97 120.65) (end 152.4 109.22) (width 0.5) (layer "B.Cu") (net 38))
 (segment (start 140.97 134.62) (end 140.97 120.65) (width 0.5) (layer "B.Cu") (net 38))
 (segment (start 143.51 120.65) (end 152.4 111.76) (width 0.5) (layer "B.Cu") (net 40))
 (segment (start 143.51 134.62) (end 143.51 120.65) (width 0.5) (layer "B.Cu") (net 40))
 (segment (start 138.43 120.65) (end 152.4 106.68) (width 0.5) (layer "B.Cu") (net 36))
 (segment (start 138.43 134.62) (end 138.43 120.65) (width 0.5) (layer "B.Cu") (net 36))
 (segment (start 113.03 137.16) (end 115.57 134.62) (width 0.5) (layer "B.Cu") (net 4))
 (segment (start 104.14 137.16) (end 113.03 137.16) (width 0.5) (layer "B.Cu") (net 4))
 (segment (start 102.87 135.89) (end 104.14 137.16) (width 0.5) (layer "B.Cu") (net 4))
 (segment (start 146.05 134.62) (end 146.05 130.81) (width 0.5) (layer "B.Cu") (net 1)))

